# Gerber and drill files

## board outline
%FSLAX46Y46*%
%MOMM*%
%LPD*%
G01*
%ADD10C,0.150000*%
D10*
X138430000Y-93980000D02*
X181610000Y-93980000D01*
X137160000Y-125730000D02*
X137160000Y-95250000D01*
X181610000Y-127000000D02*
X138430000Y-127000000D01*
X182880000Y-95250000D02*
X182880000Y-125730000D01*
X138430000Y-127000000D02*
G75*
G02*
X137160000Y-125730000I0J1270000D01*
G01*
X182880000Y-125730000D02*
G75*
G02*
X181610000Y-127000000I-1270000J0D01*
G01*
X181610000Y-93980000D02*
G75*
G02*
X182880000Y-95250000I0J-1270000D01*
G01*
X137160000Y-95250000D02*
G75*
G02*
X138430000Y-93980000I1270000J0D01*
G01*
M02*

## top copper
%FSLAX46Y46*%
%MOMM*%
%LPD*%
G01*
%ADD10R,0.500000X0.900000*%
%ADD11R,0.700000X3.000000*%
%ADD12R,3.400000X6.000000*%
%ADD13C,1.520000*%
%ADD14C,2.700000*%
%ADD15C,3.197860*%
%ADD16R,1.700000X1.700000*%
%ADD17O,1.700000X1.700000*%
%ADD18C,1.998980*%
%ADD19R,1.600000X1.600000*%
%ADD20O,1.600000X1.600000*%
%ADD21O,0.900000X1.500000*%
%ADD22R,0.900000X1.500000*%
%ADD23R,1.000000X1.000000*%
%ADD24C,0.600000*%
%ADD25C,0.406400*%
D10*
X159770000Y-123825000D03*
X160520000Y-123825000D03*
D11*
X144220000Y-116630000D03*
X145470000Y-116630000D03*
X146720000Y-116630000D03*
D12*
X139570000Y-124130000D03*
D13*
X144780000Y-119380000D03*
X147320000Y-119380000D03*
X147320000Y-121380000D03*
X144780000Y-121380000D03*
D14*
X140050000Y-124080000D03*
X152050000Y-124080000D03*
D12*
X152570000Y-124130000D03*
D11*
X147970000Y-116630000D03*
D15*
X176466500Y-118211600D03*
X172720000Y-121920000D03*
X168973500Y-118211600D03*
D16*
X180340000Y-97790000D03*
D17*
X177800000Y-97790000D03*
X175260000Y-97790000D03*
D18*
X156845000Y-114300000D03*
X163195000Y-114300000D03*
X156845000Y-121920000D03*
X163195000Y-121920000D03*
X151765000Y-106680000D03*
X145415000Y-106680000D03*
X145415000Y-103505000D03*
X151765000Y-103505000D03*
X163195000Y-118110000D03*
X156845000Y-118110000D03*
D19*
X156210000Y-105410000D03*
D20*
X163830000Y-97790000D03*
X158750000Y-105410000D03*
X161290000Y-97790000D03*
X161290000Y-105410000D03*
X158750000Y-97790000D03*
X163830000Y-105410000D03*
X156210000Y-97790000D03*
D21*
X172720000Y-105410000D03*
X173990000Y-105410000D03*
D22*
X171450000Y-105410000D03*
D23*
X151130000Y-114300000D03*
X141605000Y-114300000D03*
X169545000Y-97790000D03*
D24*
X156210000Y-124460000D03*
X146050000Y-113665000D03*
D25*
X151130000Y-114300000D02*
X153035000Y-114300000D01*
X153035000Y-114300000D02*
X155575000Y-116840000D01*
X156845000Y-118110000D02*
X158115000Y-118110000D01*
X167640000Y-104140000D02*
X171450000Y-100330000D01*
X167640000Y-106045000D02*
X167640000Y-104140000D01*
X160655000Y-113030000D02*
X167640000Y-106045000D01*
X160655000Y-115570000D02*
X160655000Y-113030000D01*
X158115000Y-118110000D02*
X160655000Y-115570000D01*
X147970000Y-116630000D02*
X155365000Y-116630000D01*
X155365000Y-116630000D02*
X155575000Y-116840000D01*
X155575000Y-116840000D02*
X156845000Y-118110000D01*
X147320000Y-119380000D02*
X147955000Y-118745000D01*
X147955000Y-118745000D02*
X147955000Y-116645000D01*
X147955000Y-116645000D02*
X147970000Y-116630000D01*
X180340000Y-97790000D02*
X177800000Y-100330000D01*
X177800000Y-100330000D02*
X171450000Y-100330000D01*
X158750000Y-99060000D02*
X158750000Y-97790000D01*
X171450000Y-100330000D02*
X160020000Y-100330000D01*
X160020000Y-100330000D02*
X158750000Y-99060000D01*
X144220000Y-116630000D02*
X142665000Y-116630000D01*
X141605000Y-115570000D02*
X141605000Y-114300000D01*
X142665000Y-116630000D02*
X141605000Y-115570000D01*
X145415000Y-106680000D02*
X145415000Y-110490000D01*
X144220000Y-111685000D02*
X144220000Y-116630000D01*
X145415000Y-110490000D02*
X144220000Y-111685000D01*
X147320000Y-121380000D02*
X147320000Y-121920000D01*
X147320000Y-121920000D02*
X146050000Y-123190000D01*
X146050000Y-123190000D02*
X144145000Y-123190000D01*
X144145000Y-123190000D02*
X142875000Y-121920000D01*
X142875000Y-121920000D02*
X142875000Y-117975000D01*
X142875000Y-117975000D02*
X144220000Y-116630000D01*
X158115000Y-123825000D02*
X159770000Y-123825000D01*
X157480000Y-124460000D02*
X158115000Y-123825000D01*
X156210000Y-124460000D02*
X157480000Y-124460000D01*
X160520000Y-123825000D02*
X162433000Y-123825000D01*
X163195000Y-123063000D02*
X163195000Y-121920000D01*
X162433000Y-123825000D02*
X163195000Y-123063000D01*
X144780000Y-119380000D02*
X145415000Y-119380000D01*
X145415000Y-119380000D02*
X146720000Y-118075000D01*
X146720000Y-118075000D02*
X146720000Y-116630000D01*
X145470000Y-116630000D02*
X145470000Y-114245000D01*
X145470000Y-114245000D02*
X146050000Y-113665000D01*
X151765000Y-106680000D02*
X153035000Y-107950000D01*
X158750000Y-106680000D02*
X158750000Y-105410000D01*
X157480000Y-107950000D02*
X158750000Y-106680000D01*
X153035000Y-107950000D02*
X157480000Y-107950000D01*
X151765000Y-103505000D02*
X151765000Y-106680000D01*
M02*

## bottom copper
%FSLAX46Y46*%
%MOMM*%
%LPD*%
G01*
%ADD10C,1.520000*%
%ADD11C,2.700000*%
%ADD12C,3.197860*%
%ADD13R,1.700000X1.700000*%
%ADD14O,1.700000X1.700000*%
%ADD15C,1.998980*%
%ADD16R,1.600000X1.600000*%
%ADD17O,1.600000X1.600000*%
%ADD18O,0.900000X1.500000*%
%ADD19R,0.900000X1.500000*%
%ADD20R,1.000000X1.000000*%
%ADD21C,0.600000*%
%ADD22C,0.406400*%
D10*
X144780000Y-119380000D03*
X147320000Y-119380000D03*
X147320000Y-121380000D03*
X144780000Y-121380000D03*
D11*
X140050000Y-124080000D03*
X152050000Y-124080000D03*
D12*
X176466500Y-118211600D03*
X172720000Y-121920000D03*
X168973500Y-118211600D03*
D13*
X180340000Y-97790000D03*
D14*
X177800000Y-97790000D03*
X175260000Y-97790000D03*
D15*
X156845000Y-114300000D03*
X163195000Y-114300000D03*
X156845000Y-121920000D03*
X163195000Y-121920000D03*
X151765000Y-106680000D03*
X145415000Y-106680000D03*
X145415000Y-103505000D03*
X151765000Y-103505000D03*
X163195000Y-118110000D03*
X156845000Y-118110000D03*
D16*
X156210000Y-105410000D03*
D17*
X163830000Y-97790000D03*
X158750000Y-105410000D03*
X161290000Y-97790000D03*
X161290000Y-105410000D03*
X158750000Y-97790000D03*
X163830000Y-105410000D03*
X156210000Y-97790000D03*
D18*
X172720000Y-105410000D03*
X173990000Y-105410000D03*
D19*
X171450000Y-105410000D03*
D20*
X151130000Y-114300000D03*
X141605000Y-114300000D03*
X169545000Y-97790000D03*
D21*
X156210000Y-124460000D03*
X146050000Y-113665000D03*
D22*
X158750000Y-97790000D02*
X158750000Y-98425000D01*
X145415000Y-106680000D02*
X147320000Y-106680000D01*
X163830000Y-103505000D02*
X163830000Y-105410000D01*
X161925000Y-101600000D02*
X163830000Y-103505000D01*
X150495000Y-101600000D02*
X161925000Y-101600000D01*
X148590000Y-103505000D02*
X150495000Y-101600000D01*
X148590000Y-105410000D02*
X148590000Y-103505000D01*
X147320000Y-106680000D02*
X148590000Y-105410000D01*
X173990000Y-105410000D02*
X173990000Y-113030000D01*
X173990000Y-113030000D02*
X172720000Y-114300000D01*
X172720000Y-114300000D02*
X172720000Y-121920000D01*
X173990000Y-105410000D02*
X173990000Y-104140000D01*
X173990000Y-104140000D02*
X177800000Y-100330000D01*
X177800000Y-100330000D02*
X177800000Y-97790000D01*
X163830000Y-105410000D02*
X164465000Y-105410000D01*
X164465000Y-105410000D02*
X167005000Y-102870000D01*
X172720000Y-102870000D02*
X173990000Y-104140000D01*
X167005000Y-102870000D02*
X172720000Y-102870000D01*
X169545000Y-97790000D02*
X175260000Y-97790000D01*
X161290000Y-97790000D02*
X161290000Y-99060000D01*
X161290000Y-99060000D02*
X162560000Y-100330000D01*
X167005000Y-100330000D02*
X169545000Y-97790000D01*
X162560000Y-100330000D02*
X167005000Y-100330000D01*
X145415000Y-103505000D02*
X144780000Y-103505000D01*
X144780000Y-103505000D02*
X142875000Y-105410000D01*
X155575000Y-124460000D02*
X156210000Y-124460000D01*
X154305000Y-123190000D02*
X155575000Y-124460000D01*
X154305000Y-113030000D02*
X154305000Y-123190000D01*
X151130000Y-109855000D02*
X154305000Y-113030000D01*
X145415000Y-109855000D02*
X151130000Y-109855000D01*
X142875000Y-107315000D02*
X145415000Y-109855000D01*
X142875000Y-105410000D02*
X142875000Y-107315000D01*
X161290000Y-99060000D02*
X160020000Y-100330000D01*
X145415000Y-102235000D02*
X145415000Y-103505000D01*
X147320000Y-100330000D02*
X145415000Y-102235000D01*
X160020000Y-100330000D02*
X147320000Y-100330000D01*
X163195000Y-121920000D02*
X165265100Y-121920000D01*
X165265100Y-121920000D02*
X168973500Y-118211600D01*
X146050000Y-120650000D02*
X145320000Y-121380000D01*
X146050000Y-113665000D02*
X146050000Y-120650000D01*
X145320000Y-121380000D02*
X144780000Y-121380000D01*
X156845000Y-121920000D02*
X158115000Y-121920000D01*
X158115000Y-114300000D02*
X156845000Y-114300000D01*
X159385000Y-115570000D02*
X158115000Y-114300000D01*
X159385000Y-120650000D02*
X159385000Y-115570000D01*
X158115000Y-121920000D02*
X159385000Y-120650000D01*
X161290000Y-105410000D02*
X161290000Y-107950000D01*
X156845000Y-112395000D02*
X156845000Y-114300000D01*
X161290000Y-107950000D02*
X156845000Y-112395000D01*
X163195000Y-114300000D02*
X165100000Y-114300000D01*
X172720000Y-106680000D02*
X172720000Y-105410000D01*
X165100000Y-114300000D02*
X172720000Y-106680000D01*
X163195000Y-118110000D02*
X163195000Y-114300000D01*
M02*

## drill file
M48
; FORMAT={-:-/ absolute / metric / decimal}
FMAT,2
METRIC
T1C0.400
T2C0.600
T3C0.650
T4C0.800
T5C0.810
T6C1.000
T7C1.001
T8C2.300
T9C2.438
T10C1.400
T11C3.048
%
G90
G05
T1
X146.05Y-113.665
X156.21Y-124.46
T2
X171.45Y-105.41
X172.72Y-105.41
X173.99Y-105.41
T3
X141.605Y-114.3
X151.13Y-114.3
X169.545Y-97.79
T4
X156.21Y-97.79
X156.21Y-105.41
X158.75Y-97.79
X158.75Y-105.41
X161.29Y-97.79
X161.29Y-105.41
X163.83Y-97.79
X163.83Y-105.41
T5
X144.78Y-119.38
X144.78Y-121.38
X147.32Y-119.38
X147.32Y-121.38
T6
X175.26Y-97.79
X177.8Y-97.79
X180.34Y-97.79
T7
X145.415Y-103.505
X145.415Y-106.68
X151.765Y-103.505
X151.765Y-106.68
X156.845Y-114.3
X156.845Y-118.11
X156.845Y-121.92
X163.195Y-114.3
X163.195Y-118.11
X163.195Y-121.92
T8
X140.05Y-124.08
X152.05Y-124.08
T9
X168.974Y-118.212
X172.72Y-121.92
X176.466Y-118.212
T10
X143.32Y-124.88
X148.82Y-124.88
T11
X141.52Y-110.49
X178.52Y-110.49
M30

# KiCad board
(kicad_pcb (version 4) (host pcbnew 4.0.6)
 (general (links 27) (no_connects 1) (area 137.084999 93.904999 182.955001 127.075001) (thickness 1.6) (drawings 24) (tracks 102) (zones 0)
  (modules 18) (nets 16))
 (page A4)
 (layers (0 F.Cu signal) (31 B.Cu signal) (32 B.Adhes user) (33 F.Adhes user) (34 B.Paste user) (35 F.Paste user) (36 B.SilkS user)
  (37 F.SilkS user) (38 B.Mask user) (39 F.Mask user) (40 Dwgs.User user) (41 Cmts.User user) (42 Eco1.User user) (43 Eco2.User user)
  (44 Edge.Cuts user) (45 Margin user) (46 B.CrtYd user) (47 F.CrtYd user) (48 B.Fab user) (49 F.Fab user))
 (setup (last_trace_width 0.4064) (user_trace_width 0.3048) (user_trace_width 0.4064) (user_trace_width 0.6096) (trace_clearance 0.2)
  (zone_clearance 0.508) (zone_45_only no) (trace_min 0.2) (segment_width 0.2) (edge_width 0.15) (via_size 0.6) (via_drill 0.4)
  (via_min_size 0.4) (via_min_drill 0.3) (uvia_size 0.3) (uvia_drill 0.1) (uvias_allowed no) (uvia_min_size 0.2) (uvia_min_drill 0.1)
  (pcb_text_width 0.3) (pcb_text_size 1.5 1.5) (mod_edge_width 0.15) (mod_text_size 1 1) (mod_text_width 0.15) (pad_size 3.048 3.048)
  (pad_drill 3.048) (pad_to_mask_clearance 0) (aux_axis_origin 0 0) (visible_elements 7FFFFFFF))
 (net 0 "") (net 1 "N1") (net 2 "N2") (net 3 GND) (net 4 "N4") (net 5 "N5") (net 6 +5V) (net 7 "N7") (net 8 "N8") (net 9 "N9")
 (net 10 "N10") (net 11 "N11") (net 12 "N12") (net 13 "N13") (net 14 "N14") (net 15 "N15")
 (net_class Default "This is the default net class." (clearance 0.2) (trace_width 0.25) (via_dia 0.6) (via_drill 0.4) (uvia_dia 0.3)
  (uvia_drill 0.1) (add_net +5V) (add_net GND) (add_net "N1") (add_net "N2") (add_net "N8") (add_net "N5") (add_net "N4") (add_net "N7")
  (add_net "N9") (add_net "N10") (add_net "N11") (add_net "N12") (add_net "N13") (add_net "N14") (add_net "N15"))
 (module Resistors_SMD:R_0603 (layer F.Cu) (at 160.02 123.825)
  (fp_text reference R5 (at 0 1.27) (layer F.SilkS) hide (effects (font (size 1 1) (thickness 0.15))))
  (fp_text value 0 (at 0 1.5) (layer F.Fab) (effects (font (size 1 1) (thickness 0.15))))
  (pad 1 smd rect (at -0.25 0) (size 0.5 0.9) (layers F.Cu F.Paste F.Mask) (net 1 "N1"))
  (pad 2 smd rect (at 0.5 0) (size 0.5 0.9) (layers F.Cu F.Paste F.Mask) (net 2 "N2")))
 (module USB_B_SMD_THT (layer F.Cu) (at 147.32 119.38 270)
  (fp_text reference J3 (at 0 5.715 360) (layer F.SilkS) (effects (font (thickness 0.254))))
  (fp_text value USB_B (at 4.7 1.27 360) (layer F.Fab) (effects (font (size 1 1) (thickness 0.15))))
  (pad 4 smd rect (at -2.75 3.1 270) (size 3 0.7) (layers F.Cu F.Paste F.Mask) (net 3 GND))
  (pad 3 smd rect (at -2.75 1.85 270) (size 3 0.7) (layers F.Cu F.Paste F.Mask) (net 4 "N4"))
  (pad 2 smd rect (at -2.75 0.6 270) (size 3 0.7) (layers F.Cu F.Paste F.Mask) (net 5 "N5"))
  (pad "" smd rect (at 4.75 7.75 270) (size 6 3.4) (layers F.Cu F.Paste F.Mask))
  (pad "" np_thru_hole circle (at 5.5 -1.5 270) (size 1.4 1.4) (drill 1.4) (layers *.Cu *.Mask))
  (pad 2 thru_hole circle (at 0 2.54 180) (size 1.52 1.52) (drill 0.81) (layers *.Cu *.Mask) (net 5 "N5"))
  (pad 1 thru_hole circle (at 0 0 180) (size 1.52 1.52) (drill 0.81) (layers *.Cu *.Mask) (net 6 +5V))
  (pad 4 thru_hole circle (at 2 0 180) (size 1.52 1.52) (drill 0.81) (layers *.Cu *.Mask) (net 3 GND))
  (pad 3 thru_hole circle (at 2 2.54 180) (size 1.52 1.52) (drill 0.81) (layers *.Cu *.Mask) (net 4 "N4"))
  (pad 5 thru_hole circle (at 4.7 7.27 180) (size 2.7 2.7) (drill 2.3) (layers *.Cu *.Mask) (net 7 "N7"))
  (pad 5 thru_hole circle (at 4.7 -4.73 180) (size 2.7 2.7) (drill 2.3) (layers *.Cu *.Mask) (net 7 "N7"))
  (pad "" np_thru_hole circle (at 5.5 4 270) (size 1.4 1.4) (drill 1.4) (layers *.Cu *.Mask))
  (pad "" smd rect (at 4.75 -5.25 270) (size 6 3.4) (layers F.Cu F.Paste F.Mask))
  (pad 1 smd rect (at -2.75 -0.65 270) (size 3 0.7) (layers F.Cu F.Paste F.Mask) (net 6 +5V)))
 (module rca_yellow (layer F.Cu) (at 172.72 121.92)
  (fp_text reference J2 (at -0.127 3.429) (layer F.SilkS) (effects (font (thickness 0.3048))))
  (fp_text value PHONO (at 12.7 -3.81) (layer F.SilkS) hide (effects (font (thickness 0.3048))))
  (pad 3 thru_hole circle (at 3.7465 -3.7084) (size 3.19786 3.19786) (drill 2.4384) (layers *.Cu *.Mask F.SilkS) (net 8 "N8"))
  (pad 1 thru_hole circle (at 0 0) (size 3.19786 3.19786) (drill 2.4384) (layers *.Cu *.Mask F.SilkS) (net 3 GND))
  (pad 2 thru_hole circle (at -3.7465 -3.7084) (size 3.19786 3.19786) (drill 2.4384) (layers *.Cu *.Mask F.SilkS) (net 2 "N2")))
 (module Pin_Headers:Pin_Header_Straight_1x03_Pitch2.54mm (layer F.Cu) (at 180.34 97.79 270)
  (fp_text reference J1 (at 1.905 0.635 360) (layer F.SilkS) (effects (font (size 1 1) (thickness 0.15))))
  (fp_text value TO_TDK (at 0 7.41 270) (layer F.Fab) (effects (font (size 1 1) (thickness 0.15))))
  (pad 1 thru_hole rect (at 0 0 270) (size 1.7 1.7) (drill 1) (layers *.Cu *.Mask) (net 6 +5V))
  (pad 2 thru_hole oval (at 0 2.54 270) (size 1.7 1.7) (drill 1) (layers *.Cu *.Mask) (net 3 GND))
  (pad 3 thru_hole oval (at 0 5.08 270) (size 1.7 1.7) (drill 1) (layers *.Cu *.Mask) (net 1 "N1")))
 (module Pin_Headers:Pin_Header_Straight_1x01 (layer F.Cu) (at 142.24 110.49)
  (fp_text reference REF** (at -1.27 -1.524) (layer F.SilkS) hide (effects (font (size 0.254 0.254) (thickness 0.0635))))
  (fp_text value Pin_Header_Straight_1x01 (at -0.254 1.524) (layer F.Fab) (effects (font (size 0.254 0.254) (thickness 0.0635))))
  (pad "" np_thru_hole circle (at -0.72 0) (size 3.048 3.048) (drill 3.048) (layers *.Cu *.Mask)))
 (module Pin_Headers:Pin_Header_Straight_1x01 (layer F.Cu) (at 177.8 110.49)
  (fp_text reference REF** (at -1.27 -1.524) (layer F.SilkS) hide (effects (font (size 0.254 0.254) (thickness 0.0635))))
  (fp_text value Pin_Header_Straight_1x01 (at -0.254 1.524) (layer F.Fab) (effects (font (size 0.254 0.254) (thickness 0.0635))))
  (pad "" np_thru_hole circle (at 0.72 0) (size 3.048 3.048) (drill 3.048) (layers *.Cu *.Mask)))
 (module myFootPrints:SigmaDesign (layer F.Cu) (at 160.02 110.49)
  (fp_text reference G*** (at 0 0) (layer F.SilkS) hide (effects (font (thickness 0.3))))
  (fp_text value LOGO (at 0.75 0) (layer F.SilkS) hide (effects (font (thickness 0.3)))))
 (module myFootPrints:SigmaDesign (layer F.Cu) (at 160.02 110.49)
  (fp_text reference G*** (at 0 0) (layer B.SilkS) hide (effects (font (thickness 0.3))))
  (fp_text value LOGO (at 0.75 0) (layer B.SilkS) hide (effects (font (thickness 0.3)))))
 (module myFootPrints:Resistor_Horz (layer F.Cu) (at 160.02 114.3)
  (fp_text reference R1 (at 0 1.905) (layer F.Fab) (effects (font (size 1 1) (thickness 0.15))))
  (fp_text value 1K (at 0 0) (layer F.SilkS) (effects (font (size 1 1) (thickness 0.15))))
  (pad 1 thru_hole circle (at -3.175 0) (size 1.99898 1.99898) (drill 1.00076) (layers *.Cu *.SilkS *.Mask) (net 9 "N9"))
  (pad 2 thru_hole circle (at 3.175 0) (size 1.99898 1.99898) (drill 1.00076) (layers *.Cu *.SilkS *.Mask) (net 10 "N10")))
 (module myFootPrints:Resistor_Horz (layer F.Cu) (at 160.02 121.92)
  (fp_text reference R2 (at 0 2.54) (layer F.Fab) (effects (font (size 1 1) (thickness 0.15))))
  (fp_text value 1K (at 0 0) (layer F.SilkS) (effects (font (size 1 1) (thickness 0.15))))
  (pad 1 thru_hole circle (at -3.175 0) (size 1.99898 1.99898) (drill 1.00076) (layers *.Cu *.SilkS *.Mask) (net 9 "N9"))
  (pad 2 thru_hole circle (at 3.175 0) (size 1.99898 1.99898) (drill 1.00076) (layers *.Cu *.SilkS *.Mask) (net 2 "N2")))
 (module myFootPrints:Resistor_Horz (layer F.Cu) (at 148.59 106.68 180)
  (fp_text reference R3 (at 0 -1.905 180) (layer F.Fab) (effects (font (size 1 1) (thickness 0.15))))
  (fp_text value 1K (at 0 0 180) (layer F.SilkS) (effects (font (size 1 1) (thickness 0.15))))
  (pad 1 thru_hole circle (at -3.175 0 180) (size 1.99898 1.99898) (drill 1.00076) (layers *.Cu *.SilkS *.Mask) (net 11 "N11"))
  (pad 2 thru_hole circle (at 3.175 0 180) (size 1.99898 1.99898) (drill 1.00076) (layers *.Cu *.SilkS *.Mask) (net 3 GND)))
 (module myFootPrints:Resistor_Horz (layer F.Cu) (at 148.59 103.505)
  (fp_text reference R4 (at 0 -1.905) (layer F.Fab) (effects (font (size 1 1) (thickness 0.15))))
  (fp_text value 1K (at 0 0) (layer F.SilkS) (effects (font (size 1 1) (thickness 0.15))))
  (pad 1 thru_hole circle (at -3.175 0) (size 1.99898 1.99898) (drill 1.00076) (layers *.Cu *.SilkS *.Mask) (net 1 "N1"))
  (pad 2 thru_hole circle (at 3.175 0) (size 1.99898 1.99898) (drill 1.00076) (layers *.Cu *.SilkS *.Mask) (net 11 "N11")))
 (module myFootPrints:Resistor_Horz (layer F.Cu) (at 160.02 118.11 180)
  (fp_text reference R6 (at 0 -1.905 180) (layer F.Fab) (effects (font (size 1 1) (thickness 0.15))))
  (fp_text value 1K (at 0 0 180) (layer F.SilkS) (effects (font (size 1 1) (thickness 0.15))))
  (pad 1 thru_hole circle (at -3.175 0 180) (size 1.99898 1.99898) (drill 1.00076) (layers *.Cu *.SilkS *.Mask) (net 10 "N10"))
  (pad 2 thru_hole circle (at 3.175 0 180) (size 1.99898 1.99898) (drill 1.00076) (layers *.Cu *.SilkS *.Mask) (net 6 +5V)))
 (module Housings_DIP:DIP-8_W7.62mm (layer F.Cu) (at 156.21 105.41 90)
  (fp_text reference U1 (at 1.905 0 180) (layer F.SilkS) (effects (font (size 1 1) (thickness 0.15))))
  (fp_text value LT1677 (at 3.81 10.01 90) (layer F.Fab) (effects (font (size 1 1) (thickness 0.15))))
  (pad 1 thru_hole rect (at 0 0 90) (size 1.6 1.6) (drill 0.8) (layers *.Cu *.Mask) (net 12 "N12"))
  (pad 5 thru_hole oval (at 7.62 7.62 90) (size 1.6 1.6) (drill 0.8) (layers *.Cu *.Mask) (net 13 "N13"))
  (pad 2 thru_hole oval (at 0 2.54 90) (size 1.6 1.6) (drill 0.8) (layers *.Cu *.Mask) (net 11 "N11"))
  (pad 6 thru_hole oval (at 7.62 5.08 90) (size 1.6 1.6) (drill 0.8) (layers *.Cu *.Mask) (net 1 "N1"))
  (pad 3 thru_hole oval (at 0 5.08 90) (size 1.6 1.6) (drill 0.8) (layers *.Cu *.Mask) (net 9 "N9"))
  (pad 7 thru_hole oval (at 7.62 2.54 90) (size 1.6 1.6) (drill 0.8) (layers *.Cu *.Mask) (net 6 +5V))
  (pad 4 thru_hole oval (at 0 7.62 90) (size 1.6 1.6) (drill 0.8) (layers *.Cu *.Mask) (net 3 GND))
  (pad 8 thru_hole oval (at 7.62 0 90) (size 1.6 1.6) (drill 0.8) (layers *.Cu *.Mask) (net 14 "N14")))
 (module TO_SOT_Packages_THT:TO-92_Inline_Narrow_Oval (layer F.Cu) (at 171.45 105.41)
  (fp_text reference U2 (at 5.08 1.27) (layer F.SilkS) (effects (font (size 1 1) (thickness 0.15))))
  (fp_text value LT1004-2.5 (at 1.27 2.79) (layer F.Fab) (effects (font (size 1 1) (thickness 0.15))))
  (pad 2 thru_hole oval (at 1.27 0 180) (size 0.9 1.5) (drill 0.6) (layers *.Cu *.Mask) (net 10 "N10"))
  (pad 3 thru_hole oval (at 2.54 0 180) (size 0.9 1.5) (drill 0.6) (layers *.Cu *.Mask) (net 3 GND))
  (pad 1 thru_hole rect (at 0 0 180) (size 0.9 1.5) (drill 0.6) (layers *.Cu *.Mask) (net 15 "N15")))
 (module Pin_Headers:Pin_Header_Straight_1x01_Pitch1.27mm (layer F.Cu) (at 151.13 114.3)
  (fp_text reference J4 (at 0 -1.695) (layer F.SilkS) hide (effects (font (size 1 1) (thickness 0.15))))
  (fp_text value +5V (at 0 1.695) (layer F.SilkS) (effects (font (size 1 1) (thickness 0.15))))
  (pad 1 thru_hole rect (at 0 0) (size 1 1) (drill 0.65) (layers *.Cu *.Mask) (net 6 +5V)))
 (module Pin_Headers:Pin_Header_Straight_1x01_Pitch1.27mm (layer F.Cu) (at 141.605 114.3)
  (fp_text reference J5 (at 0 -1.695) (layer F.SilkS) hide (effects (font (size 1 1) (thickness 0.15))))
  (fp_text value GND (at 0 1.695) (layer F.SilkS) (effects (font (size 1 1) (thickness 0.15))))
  (pad 1 thru_hole rect (at 0 0) (size 1 1) (drill 0.65) (layers *.Cu *.Mask) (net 3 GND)))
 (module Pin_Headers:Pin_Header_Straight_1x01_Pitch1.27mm (layer F.Cu) (at 169.545 97.79)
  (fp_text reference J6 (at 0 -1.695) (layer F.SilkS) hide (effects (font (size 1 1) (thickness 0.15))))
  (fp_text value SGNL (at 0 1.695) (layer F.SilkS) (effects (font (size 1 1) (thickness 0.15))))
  (pad 1 thru_hole rect (at 0 0) (size 1 1) (drill 0.65) (layers *.Cu *.Mask) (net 1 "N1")))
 (gr_line (start 138.43 93.98) (end 181.61 93.98) (angle 90) (layer Edge.Cuts) (width 0.15))
 (gr_line (start 137.16 125.73) (end 137.16 95.25) (angle 90) (layer Edge.Cuts) (width 0.15))
 (gr_line (start 181.61 127) (end 138.43 127) (angle 90) (layer Edge.Cuts) (width 0.15))
 (gr_line (start 182.88 95.25) (end 182.88 125.73) (angle 90) (layer Edge.Cuts) (width 0.15))
 (gr_arc (start 138.43 125.73) (end 138.43 127) (angle 90) (layer Edge.Cuts) (width 0.15))
 (gr_arc (start 181.61 125.73) (end 182.88 125.73) (angle 90) (layer Edge.Cuts) (width 0.15))
 (gr_arc (start 181.61 95.25) (end 181.61 93.98) (angle 90) (layer Edge.Cuts) (width 0.15))
 (gr_arc (start 138.43 95.25) (end 137.16 95.25) (angle 90) (layer Edge.Cuts) (width 0.15))
 (segment (start 151.13 114.3) (end 153.035 114.3) (width 0.4064) (layer F.Cu) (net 6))
 (segment (start 153.035 114.3) (end 155.575 116.84) (width 0.4064) (layer F.Cu) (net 6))
 (segment (start 156.845 118.11) (end 158.115 118.11) (width 0.4064) (layer F.Cu) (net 6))
 (segment (start 167.64 104.14) (end 171.45 100.33) (width 0.4064) (layer F.Cu) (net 6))
 (segment (start 167.64 106.045) (end 167.64 104.14) (width 0.4064) (layer F.Cu) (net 6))
 (segment (start 160.655 113.03) (end 167.64 106.045) (width 0.4064) (layer F.Cu) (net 6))
 (segment (start 160.655 115.57) (end 160.655 113.03) (width 0.4064) (layer F.Cu) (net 6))
 (segment (start 158.115 118.11) (end 160.655 115.57) (width 0.4064) (layer F.Cu) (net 6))
 (segment (start 147.97 116.63) (end 155.365 116.63) (width 0.4064) (layer F.Cu) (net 6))
 (segment (start 155.365 116.63) (end 155.575 116.84) (width 0.4064) (layer F.Cu) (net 6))
 (segment (start 155.575 116.84) (end 156.845 118.11) (width 0.4064) (layer F.Cu) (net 6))
 (segment (start 147.32 119.38) (end 147.955 118.745) (width 0.4064) (layer F.Cu) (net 6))
 (segment (start 147.955 118.745) (end 147.955 116.645) (width 0.4064) (layer F.Cu) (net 6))
 (segment (start 147.955 116.645) (end 147.97 116.63) (width 0.4064) (layer F.Cu) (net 6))
 (segment (start 180.34 97.79) (end 177.8 100.33) (width 0.4064) (layer F.Cu) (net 6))
 (segment (start 177.8 100.33) (end 171.45 100.33) (width 0.4064) (layer F.Cu) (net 6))
 (segment (start 158.75 99.06) (end 158.75 97.79) (width 0.4064) (layer F.Cu) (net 6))
 (segment (start 171.45 100.33) (end 160.02 100.33) (width 0.4064) (layer F.Cu) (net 6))
 (segment (start 160.02 100.33) (end 158.75 99.06) (width 0.4064) (layer F.Cu) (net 6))
 (segment (start 158.75 97.79) (end 158.75 98.425) (width 0.4064) (layer B.Cu) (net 6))
 (segment (start 144.22 116.63) (end 142.665 116.63) (width 0.4064) (layer F.Cu) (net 3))
 (segment (start 141.605 115.57) (end 141.605 114.3) (width 0.4064) (layer F.Cu) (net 3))
 (segment (start 142.665 116.63) (end 141.605 115.57) (width 0.4064) (layer F.Cu) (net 3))
 (segment (start 145.415 106.68) (end 147.32 106.68) (width 0.4064) (layer B.Cu) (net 3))
 (segment (start 163.83 103.505) (end 163.83 105.41) (width 0.4064) (layer B.Cu) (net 3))
 (segment (start 161.925 101.6) (end 163.83 103.505) (width 0.4064) (layer B.Cu) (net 3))
 (segment (start 150.495 101.6) (end 161.925 101.6) (width 0.4064) (layer B.Cu) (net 3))
 (segment (start 148.59 103.505) (end 150.495 101.6) (width 0.4064) (layer B.Cu) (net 3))
 (segment (start 148.59 105.41) (end 148.59 103.505) (width 0.4064) (layer B.Cu) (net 3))
 (segment (start 147.32 106.68) (end 148.59 105.41) (width 0.4064) (layer B.Cu) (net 3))
 (segment (start 145.415 106.68) (end 145.415 110.49) (width 0.4064) (layer F.Cu) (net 3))
 (segment (start 144.22 111.685) (end 144.22 116.63) (width 0.4064) (layer F.Cu) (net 3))
 (segment (start 145.415 110.49) (end 144.22 111.685) (width 0.4064) (layer F.Cu) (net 3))
 (segment (start 147.32 121.38) (end 147.32 121.92) (width 0.4064) (layer F.Cu) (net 3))
 (segment (start 147.32 121.92) (end 146.05 123.19) (width 0.4064) (layer F.Cu) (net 3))
 (segment (start 146.05 123.19) (end 144.145 123.19) (width 0.4064) (layer F.Cu) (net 3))
 (segment (start 144.145 123.19) (end 142.875 121.92) (width 0.4064) (layer F.Cu) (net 3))
 (segment (start 142.875 121.92) (end 142.875 117.975) (width 0.4064) (layer F.Cu) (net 3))
 (segment (start 142.875 117.975) (end 144.22 116.63) (width 0.4064) (layer F.Cu) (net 3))
 (segment (start 173.99 105.41) (end 173.99 113.03) (width 0.4064) (layer B.Cu) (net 3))
 (segment (start 173.99 113.03) (end 172.72 114.3) (width 0.4064) (layer B.Cu) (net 3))
 (segment (start 172.72 114.3) (end 172.72 121.92) (width 0.4064) (layer B.Cu) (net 3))
 (segment (start 173.99 105.41) (end 173.99 104.14) (width 0.4064) (layer B.Cu) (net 3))
 (segment (start 173.99 104.14) (end 177.8 100.33) (width 0.4064) (layer B.Cu) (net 3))
 (segment (start 177.8 100.33) (end 177.8 97.79) (width 0.4064) (layer B.Cu) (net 3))
 (segment (start 163.83 105.41) (end 164.465 105.41) (width 0.4064) (layer B.Cu) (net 3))
 (segment (start 164.465 105.41) (end 167.005 102.87) (width 0.4064) (layer B.Cu) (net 3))
 (segment (start 172.72 102.87) (end 173.99 104.14) (width 0.4064) (layer B.Cu) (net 3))
 (segment (start 167.005 102.87) (end 172.72 102.87) (width 0.4064) (layer B.Cu) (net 3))
 (segment (start 169.545 97.79) (end 175.26 97.79) (width 0.4064) (layer B.Cu) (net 1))
 (segment (start 161.29 97.79) (end 161.29 99.06) (width 0.4064) (layer B.Cu) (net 1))
 (segment (start 161.29 99.06) (end 162.56 100.33) (width 0.4064) (layer B.Cu) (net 1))
 (segment (start 167.005 100.33) (end 169.545 97.79) (width 0.4064) (layer B.Cu) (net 1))
 (segment (start 162.56 100.33) (end 167.005 100.33) (width 0.4064) (layer B.Cu) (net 1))
 (segment (start 145.415 103.505) (end 144.78 103.505) (width 0.4064) (layer B.Cu) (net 1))
 (segment (start 144.78 103.505) (end 142.875 105.41) (width 0.4064) (layer B.Cu) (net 1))
 (segment (start 158.115 123.825) (end 159.77 123.825) (width 0.4064) (layer F.Cu) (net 1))
 (segment (start 157.48 124.46) (end 158.115 123.825) (width 0.4064) (layer F.Cu) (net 1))
 (segment (start 156.21 124.46) (end 157.48 124.46) (width 0.4064) (layer F.Cu) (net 1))
 (via (at 156.21 124.46) (size 0.6) (drill 0.4) (layers F.Cu B.Cu) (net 1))
 (segment (start 155.575 124.46) (end 156.21 124.46) (width 0.4064) (layer B.Cu) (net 1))
 (segment (start 154.305 123.19) (end 155.575 124.46) (width 0.4064) (layer B.Cu) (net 1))
 (segment (start 154.305 113.03) (end 154.305 123.19) (width 0.4064) (layer B.Cu) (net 1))
 (segment (start 151.13 109.855) (end 154.305 113.03) (width 0.4064) (layer B.Cu) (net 1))
 (segment (start 145.415 109.855) (end 151.13 109.855) (width 0.4064) (layer B.Cu) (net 1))
 (segment (start 142.875 107.315) (end 145.415 109.855) (width 0.4064) (layer B.Cu) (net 1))
 (segment (start 142.875 105.41) (end 142.875 107.315) (width 0.4064) (layer B.Cu) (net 1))
 (segment (start 161.29 99.06) (end 160.02 100.33) (width 0.4064) (layer B.Cu) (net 1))
 (segment (start 145.415 102.235) (end 145.415 103.505) (width 0.4064) (layer B.Cu) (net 1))
 (segment (start 147.32 100.33) (end 145.415 102.235) (width 0.4064) (layer B.Cu) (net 1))
 (segment (start 160.02 100.33) (end 147.32 100.33) (width 0.4064) (layer B.Cu) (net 1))
 (segment (start 160.52 123.825) (end 162.433 123.825) (width 0.4064) (layer F.Cu) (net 2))
 (segment (start 163.195 123.063) (end 163.195 121.92) (width 0.4064) (layer F.Cu) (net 2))
 (segment (start 162.433 123.825) (end 163.195 123.063) (width 0.4064) (layer F.Cu) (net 2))
 (segment (start 163.195 121.92) (end 165.2651 121.92) (width 0.4064) (layer B.Cu) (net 2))
 (segment (start 165.2651 121.92) (end 168.9735 118.2116) (width 0.4064) (layer B.Cu) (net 2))
 (segment (start 144.78 119.38) (end 145.415 119.38) (width 0.4064) (layer F.Cu) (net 5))
 (segment (start 145.415 119.38) (end 146.72 118.075) (width 0.4064) (layer F.Cu) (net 5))
 (segment (start 146.72 118.075) (end 146.72 116.63) (width 0.4064) (layer F.Cu) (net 5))
 (segment (start 145.47 116.63) (end 145.47 114.245) (width 0.4064) (layer F.Cu) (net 4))
 (segment (start 146.05 120.65) (end 145.32 121.38) (width 0.4064) (layer B.Cu) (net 4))
 (segment (start 146.05 113.665) (end 146.05 120.65) (width 0.4064) (layer B.Cu) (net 4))
 (via (at 146.05 113.665) (size 0.6) (drill 0.4) (layers F.Cu B.Cu) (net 4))
 (segment (start 145.47 114.245) (end 146.05 113.665) (width 0.4064) (layer F.Cu) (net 4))
 (segment (start 145.32 121.38) (end 144.78 121.38) (width 0.4064) (layer B.Cu) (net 4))
 (segment (start 156.845 121.92) (end 158.115 121.92) (width 0.4064) (layer B.Cu) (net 9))
 (segment (start 158.115 114.3) (end 156.845 114.3) (width 0.4064) (layer B.Cu) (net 9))
 (segment (start 159.385 115.57) (end 158.115 114.3) (width 0.4064) (layer B.Cu) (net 9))
 (segment (start 159.385 120.65) (end 159.385 115.57) (width 0.4064) (layer B.Cu) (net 9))
 (segment (start 158.115 121.92) (end 159.385 120.65) (width 0.4064) (layer B.Cu) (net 9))
 (segment (start 161.29 105.41) (end 161.29 107.95) (width 0.4064) (layer B.Cu) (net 9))
 (segment (start 156.845 112.395) (end 156.845 114.3) (width 0.4064) (layer B.Cu) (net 9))
 (segment (start 161.29 107.95) (end 156.845 112.395) (width 0.4064) (layer B.Cu) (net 9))
 (segment (start 163.195 114.3) (end 165.1 114.3) (width 0.4064) (layer B.Cu) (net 10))
 (segment (start 172.72 106.68) (end 172.72 105.41) (width 0.4064) (layer B.Cu) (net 10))
 (segment (start 165.1 114.3) (end 172.72 106.68) (width 0.4064) (layer B.Cu) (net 10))
 (segment (start 163.195 118.11) (end 163.195 114.3) (width 0.4064) (layer B.Cu) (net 10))
 (segment (start 151.765 106.68) (end 153.035 107.95) (width 0.4064) (layer F.Cu) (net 11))
 (segment (start 158.75 106.68) (end 158.75 105.41) (width 0.4064) (layer F.Cu) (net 11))
 (segment (start 157.48 107.95) (end 158.75 106.68) (width 0.4064) (layer F.Cu) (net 11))
 (segment (start 153.035 107.95) (end 157.48 107.95) (width 0.4064) (layer F.Cu) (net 11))
 (segment (start 151.765 103.505) (end 151.765 106.68) (width 0.4064) (layer F.Cu) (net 11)))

